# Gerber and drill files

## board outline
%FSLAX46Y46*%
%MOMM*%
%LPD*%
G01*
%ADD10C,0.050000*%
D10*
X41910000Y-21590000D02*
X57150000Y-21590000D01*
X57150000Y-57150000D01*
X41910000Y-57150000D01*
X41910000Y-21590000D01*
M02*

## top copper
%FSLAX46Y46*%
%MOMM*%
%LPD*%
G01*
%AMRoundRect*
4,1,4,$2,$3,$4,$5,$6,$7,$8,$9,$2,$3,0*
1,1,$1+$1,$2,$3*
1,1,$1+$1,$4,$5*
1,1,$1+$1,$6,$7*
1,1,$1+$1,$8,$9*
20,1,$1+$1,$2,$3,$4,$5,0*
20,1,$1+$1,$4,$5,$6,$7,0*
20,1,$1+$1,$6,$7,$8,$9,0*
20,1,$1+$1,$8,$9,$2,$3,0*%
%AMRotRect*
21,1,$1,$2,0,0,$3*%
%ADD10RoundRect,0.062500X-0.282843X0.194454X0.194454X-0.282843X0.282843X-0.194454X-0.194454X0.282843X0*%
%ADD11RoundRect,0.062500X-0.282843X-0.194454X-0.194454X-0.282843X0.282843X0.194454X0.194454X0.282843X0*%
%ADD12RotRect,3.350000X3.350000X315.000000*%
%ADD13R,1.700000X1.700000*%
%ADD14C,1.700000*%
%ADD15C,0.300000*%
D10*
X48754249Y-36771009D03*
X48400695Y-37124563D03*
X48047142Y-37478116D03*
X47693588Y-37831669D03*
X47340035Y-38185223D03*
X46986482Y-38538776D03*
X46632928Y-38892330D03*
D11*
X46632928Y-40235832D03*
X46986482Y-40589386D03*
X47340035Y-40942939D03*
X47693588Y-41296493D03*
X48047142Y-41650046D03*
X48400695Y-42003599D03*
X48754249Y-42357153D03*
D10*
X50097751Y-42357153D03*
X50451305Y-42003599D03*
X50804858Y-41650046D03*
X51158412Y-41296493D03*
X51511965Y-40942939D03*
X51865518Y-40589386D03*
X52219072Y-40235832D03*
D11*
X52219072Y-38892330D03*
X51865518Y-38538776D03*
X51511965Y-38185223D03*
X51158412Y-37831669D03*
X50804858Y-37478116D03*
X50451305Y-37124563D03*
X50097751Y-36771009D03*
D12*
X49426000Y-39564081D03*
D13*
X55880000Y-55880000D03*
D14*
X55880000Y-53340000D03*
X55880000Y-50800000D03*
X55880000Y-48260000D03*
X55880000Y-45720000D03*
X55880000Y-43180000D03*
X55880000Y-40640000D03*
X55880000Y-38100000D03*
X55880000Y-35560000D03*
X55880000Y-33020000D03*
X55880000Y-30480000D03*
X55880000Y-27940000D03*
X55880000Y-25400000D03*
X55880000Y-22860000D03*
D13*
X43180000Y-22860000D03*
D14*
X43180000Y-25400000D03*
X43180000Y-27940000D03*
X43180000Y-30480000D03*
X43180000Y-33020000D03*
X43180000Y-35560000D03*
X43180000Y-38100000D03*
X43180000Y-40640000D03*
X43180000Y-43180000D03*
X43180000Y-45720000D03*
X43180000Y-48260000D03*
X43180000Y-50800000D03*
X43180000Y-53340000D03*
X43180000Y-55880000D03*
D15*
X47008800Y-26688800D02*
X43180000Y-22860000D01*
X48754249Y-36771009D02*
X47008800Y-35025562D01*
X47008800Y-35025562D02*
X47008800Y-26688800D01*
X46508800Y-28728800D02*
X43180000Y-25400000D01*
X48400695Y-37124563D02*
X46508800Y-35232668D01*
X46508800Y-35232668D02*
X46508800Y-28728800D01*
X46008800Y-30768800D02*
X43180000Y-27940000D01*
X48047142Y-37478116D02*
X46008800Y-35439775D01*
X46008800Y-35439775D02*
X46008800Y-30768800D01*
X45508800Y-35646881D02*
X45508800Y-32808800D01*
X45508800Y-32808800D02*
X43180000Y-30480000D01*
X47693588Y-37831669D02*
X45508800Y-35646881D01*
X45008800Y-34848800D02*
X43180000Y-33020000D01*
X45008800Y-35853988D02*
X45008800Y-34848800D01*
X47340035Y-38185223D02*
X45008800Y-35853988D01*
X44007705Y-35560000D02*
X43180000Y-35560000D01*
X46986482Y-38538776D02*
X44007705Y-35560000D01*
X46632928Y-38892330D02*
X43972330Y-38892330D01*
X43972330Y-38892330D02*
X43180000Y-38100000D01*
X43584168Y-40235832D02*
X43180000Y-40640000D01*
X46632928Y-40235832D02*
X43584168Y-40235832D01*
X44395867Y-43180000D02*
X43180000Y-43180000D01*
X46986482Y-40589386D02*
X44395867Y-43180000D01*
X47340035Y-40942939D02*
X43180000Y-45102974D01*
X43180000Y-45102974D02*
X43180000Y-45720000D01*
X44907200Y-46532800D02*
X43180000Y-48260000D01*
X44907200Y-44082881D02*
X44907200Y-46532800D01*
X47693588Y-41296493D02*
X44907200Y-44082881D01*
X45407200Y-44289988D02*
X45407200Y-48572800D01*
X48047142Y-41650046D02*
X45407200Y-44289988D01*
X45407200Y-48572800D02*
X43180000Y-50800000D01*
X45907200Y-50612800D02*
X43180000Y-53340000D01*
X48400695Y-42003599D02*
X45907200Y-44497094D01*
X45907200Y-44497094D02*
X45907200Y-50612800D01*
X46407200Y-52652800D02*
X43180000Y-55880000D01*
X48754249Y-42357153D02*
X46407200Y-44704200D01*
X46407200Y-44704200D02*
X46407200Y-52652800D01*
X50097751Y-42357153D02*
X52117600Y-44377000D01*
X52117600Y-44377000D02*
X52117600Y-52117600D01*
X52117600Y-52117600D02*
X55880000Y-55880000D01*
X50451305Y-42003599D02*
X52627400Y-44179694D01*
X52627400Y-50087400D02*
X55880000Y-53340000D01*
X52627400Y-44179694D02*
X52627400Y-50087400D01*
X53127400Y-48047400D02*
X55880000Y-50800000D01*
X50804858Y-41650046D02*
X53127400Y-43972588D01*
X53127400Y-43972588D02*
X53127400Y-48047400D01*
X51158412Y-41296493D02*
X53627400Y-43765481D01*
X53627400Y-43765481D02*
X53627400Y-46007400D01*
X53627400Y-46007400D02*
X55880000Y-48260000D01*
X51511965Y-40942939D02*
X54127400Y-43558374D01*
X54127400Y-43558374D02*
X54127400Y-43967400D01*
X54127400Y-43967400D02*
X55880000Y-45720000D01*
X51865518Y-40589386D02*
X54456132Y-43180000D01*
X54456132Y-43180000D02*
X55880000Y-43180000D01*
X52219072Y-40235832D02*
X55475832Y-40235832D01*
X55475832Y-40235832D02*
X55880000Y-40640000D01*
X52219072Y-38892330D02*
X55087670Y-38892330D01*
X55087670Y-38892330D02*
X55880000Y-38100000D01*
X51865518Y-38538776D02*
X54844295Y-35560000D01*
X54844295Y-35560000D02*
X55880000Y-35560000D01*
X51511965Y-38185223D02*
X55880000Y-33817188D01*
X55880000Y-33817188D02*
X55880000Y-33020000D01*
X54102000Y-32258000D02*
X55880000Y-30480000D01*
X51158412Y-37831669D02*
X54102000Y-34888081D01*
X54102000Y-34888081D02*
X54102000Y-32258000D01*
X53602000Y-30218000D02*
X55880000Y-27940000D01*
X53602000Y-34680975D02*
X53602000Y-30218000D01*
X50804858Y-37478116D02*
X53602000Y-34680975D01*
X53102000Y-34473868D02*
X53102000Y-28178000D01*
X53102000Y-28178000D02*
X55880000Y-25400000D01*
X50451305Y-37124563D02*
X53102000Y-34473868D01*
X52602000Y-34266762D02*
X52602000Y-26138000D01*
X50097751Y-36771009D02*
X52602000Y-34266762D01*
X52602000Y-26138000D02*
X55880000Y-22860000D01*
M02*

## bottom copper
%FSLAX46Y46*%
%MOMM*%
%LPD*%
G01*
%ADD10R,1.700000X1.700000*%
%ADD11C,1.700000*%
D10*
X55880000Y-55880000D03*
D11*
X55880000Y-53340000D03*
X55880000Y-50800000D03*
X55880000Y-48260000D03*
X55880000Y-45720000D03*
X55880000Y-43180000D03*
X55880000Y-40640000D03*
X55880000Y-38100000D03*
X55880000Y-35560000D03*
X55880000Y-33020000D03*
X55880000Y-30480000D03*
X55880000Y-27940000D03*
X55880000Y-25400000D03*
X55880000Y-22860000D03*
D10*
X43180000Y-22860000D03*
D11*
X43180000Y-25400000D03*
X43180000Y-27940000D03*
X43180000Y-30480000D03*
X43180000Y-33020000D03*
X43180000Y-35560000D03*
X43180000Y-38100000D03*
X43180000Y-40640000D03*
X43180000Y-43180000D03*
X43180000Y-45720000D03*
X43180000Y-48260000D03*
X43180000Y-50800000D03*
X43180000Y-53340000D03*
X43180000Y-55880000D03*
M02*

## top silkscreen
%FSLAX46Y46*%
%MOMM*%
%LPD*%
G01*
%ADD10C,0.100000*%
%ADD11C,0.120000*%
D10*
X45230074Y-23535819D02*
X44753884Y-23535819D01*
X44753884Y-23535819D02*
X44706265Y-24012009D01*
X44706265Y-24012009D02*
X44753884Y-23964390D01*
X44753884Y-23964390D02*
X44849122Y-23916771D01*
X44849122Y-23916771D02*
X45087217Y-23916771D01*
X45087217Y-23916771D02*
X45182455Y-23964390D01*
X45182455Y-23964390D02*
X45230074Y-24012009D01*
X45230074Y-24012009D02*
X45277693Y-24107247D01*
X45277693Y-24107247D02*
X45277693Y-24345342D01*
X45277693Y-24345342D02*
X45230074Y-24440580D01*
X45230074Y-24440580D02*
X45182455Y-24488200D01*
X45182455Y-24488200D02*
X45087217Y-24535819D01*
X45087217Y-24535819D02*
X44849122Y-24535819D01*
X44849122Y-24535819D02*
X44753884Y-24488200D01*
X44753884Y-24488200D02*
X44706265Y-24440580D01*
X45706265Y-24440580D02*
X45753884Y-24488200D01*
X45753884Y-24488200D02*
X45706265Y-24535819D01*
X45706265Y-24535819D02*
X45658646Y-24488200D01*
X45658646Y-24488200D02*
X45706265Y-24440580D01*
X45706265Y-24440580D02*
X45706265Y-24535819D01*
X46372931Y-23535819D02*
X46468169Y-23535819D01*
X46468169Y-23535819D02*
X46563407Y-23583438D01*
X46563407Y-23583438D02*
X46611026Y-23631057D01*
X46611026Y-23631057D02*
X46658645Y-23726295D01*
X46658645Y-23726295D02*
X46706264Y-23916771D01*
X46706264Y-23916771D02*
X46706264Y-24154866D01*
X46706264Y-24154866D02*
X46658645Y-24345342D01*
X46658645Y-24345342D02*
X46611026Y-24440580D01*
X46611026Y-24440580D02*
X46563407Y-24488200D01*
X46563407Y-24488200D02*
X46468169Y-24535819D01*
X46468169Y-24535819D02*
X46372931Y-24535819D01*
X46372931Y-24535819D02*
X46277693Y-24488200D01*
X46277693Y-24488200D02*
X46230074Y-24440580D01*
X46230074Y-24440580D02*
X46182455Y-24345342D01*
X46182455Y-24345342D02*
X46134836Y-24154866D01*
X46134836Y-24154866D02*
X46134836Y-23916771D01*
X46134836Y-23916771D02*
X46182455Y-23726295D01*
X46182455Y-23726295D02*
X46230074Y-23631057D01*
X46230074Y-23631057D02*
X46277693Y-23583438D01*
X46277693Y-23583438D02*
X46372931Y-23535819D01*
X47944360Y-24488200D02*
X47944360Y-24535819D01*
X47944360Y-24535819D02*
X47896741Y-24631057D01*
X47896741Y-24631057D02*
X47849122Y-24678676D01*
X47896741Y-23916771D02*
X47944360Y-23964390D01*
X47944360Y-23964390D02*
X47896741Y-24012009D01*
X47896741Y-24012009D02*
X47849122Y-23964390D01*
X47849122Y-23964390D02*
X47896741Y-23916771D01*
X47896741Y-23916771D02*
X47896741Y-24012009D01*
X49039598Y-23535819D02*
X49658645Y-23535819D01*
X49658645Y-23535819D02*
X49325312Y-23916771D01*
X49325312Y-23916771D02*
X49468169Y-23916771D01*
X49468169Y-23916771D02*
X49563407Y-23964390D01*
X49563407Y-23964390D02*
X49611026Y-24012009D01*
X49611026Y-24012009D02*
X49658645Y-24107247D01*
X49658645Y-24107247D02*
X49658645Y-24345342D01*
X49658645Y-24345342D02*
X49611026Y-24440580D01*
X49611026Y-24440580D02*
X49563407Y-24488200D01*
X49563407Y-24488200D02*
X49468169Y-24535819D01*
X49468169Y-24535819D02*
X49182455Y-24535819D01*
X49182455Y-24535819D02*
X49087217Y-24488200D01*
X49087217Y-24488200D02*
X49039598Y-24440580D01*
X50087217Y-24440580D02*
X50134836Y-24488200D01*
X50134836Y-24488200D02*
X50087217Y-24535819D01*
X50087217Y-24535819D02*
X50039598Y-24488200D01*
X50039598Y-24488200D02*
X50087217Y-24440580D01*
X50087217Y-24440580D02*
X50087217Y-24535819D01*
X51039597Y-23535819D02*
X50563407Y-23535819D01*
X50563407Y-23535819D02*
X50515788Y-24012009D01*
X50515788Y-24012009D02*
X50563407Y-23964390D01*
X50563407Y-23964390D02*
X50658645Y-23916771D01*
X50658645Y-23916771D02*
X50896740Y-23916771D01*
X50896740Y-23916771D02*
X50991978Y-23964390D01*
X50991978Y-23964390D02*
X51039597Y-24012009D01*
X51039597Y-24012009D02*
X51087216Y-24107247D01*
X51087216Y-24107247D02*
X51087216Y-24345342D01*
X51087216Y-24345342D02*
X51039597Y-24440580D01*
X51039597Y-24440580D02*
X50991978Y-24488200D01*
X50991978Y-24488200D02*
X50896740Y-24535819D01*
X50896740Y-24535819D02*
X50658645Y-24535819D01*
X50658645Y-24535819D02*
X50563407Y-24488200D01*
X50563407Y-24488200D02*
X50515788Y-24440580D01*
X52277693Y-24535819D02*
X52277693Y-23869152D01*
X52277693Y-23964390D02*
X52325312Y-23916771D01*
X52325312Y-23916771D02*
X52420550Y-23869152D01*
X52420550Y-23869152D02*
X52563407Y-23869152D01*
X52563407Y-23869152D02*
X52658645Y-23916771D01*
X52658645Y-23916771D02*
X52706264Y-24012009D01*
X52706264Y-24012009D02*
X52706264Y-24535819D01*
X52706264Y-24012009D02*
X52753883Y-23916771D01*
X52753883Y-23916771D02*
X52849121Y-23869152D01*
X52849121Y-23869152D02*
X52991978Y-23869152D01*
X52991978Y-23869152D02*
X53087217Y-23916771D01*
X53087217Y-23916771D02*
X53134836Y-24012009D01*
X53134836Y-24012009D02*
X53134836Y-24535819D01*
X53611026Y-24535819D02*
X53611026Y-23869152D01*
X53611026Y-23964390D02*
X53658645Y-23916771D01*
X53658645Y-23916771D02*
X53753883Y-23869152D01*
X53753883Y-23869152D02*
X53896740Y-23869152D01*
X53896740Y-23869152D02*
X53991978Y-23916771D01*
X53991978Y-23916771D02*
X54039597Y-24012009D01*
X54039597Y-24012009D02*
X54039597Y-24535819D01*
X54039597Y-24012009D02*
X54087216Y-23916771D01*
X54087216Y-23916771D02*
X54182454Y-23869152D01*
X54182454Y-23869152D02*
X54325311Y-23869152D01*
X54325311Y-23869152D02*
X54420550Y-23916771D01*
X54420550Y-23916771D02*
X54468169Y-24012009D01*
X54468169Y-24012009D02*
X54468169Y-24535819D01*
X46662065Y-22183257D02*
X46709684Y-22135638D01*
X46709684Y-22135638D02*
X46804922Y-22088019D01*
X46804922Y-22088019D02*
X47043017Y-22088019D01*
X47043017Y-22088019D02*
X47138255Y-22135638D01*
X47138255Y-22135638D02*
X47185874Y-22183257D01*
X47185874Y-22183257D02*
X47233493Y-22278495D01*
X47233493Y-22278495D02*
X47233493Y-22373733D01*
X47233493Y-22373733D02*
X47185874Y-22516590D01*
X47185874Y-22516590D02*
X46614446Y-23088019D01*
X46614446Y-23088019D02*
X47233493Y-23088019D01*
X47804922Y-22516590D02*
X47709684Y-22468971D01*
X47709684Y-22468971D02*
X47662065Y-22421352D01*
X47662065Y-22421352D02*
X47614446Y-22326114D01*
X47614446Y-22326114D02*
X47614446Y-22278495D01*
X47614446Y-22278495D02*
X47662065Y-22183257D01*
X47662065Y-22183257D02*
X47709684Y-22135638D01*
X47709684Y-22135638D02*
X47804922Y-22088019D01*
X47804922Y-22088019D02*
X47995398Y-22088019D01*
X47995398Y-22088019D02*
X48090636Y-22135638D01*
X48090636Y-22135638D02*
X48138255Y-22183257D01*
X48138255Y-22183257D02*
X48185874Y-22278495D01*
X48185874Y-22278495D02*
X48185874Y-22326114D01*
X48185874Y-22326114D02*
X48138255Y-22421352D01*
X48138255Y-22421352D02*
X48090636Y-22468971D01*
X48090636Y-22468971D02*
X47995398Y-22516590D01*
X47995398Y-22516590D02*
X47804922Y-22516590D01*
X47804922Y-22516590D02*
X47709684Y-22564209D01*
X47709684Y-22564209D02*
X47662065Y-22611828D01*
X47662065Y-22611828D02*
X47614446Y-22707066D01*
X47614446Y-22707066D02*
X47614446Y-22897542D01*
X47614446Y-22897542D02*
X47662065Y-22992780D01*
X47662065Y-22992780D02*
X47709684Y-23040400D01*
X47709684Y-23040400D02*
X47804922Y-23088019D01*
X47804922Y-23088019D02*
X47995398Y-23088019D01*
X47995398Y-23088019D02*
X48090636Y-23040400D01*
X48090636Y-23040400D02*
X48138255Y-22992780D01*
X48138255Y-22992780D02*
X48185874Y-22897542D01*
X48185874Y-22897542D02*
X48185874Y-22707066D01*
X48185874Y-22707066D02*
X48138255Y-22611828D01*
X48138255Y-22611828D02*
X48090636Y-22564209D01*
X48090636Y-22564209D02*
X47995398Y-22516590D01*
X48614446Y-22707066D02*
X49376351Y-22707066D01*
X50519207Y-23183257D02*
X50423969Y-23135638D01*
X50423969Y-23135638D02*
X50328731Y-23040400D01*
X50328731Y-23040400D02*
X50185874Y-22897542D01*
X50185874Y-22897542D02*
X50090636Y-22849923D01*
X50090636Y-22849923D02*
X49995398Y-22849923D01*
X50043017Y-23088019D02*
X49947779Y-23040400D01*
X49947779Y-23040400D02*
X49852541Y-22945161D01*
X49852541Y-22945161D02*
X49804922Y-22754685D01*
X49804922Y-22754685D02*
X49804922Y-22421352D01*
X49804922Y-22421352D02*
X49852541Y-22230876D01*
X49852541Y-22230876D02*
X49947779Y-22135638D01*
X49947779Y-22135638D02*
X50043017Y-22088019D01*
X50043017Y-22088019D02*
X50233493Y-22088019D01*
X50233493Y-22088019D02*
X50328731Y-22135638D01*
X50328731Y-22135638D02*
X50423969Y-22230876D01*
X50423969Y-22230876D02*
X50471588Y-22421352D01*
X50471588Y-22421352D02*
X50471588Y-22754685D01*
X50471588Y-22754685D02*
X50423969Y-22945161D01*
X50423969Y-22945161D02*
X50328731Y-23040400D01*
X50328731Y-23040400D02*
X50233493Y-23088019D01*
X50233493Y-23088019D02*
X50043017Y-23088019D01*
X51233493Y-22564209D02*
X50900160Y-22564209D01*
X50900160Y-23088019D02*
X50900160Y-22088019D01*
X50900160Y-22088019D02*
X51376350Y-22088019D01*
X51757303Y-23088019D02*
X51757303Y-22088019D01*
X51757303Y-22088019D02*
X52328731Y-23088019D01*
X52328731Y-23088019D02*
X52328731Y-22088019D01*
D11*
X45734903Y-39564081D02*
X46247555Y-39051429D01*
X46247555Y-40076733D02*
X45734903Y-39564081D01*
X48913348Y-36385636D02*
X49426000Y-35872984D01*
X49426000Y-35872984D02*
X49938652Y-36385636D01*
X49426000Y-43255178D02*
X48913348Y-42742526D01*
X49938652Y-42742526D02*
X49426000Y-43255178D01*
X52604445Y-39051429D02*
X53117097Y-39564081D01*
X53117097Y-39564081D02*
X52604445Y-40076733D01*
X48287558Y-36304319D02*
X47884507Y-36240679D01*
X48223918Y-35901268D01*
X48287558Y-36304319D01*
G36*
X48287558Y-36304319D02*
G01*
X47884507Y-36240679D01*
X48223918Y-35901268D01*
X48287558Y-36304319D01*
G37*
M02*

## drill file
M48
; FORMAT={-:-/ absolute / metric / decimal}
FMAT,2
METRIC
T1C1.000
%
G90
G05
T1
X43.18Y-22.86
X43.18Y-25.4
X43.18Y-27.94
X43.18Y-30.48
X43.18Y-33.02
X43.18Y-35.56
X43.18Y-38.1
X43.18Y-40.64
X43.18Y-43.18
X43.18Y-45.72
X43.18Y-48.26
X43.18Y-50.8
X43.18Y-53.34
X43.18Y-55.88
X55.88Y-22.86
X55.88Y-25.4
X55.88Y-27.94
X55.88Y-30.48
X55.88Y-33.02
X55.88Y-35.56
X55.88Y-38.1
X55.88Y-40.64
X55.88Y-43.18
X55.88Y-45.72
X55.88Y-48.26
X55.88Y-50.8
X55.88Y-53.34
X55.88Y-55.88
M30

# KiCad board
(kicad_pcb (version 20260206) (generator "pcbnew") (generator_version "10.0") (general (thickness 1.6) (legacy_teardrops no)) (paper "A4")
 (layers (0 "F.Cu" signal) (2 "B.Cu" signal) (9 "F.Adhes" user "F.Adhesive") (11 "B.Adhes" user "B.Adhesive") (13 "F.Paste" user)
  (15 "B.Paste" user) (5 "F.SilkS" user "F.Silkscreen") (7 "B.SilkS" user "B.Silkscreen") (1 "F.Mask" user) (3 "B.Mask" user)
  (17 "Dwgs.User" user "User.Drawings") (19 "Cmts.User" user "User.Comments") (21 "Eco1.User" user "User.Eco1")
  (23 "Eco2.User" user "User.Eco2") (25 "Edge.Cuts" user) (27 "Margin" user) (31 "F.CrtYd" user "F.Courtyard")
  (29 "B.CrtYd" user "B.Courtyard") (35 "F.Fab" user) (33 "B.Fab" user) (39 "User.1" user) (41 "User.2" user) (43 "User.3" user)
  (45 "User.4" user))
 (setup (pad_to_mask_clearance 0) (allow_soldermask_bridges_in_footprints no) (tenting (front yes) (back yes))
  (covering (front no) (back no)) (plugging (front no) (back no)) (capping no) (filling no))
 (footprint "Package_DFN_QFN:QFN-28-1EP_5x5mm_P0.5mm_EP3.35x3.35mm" (layer "F.Cu") (at 49.426 39.564081 -45)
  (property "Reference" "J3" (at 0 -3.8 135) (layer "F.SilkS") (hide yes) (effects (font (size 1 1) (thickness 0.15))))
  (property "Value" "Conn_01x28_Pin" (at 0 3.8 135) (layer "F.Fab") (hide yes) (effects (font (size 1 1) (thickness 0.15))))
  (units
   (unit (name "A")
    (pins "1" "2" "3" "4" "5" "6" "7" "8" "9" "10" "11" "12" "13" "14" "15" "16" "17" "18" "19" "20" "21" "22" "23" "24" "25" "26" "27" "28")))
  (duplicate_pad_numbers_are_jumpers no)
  (fp_line (start -2.61 2.61) (end -2.61 1.885) (stroke (width 0.12) (type solid)) (layer "F.SilkS"))
  (fp_line (start -1.885 2.61) (end -2.61 2.61) (stroke (width 0.12) (type solid)) (layer "F.SilkS"))
  (fp_line (start -2.61 -1.885) (end -2.61 -2.61) (stroke (width 0.12) (type solid)) (layer "F.SilkS"))
  (fp_line (start -2.61 -2.61) (end -1.885 -2.61) (stroke (width 0.12) (type solid)) (layer "F.SilkS"))
  (fp_line (start 2.61 2.61) (end 1.885 2.61) (stroke (width 0.12) (type solid)) (layer "F.SilkS"))
  (fp_line (start 2.61 1.885) (end 2.61 2.61) (stroke (width 0.12) (type solid)) (layer "F.SilkS"))
  (fp_line (start 1.885 -2.61) (end 2.61 -2.61) (stroke (width 0.12) (type solid)) (layer "F.SilkS"))
  (fp_line (start 2.61 -2.61) (end 2.61 -1.885) (stroke (width 0.12) (type solid)) (layer "F.SilkS"))
  (fp_poly (pts (xy -3.11 -1.5) (xy -3.44 -1.26) (xy -3.44 -1.74)) (stroke (width 0.12) (type solid)) (fill yes) (layer "F.SilkS"))
  (pad "" smd roundrect (at -1.120001 0 315) (size 0.9 0.9) (layers "F.Paste") (roundrect_rratio 0.25))
  (pad "" smd roundrect (at -1.12 -1.12 315) (size 0.9 0.9) (layers "F.Paste") (roundrect_rratio 0.25))
  (pad "" smd roundrect (at -1.12 1.12 315) (size 0.9 0.9) (layers "F.Paste") (roundrect_rratio 0.25))
  (pad "" smd roundrect (at 0 -1.120001 315) (size 0.9 0.9) (layers "F.Paste") (roundrect_rratio 0.25))
  (pad "" smd roundrect (at 0 0 315) (size 0.9 0.9) (layers "F.Paste") (roundrect_rratio 0.25))
  (pad "" smd roundrect (at 0 1.120001 315) (size 0.9 0.9) (layers "F.Paste") (roundrect_rratio 0.25))
  (pad "" smd roundrect (at 1.12 -1.12 315) (size 0.9 0.9) (layers "F.Paste") (roundrect_rratio 0.25))
  (pad "" smd roundrect (at 1.12 1.12 315) (size 0.9 0.9) (layers "F.Paste") (roundrect_rratio 0.25))
  (pad "" smd roundrect (at 1.120001 0 315) (size 0.9 0.9) (layers "F.Paste") (roundrect_rratio 0.25))
  (pad "1" smd roundrect (at -2.45 -1.5 315) (size 0.8 0.25) (layers "F.Cu" "F.Mask" "F.Paste") (roundrect_rratio 0.25)
   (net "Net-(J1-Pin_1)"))
  (pad "2" smd roundrect (at -2.45 -1 315) (size 0.8 0.25) (layers "F.Cu" "F.Mask" "F.Paste") (roundrect_rratio 0.25) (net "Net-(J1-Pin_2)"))
  (pad "3" smd roundrect (at -2.45 -0.5 315) (size 0.8 0.25) (layers "F.Cu" "F.Mask" "F.Paste") (roundrect_rratio 0.25)
   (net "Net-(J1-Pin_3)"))
  (pad "4" smd roundrect (at -2.450001 0 315) (size 0.8 0.25) (layers "F.Cu" "F.Mask" "F.Paste") (roundrect_rratio 0.25)
   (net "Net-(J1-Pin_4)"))
  (pad "5" smd roundrect (at -2.45 0.5 315) (size 0.8 0.25) (layers "F.Cu" "F.Mask" "F.Paste") (roundrect_rratio 0.25)
   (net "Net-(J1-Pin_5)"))
  (pad "6" smd roundrect (at -2.45 1 315) (size 0.8 0.25) (layers "F.Cu" "F.Mask" "F.Paste") (roundrect_rratio 0.25) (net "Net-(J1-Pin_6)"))
  (pad "7" smd roundrect (at -2.45 1.5 315) (size 0.8 0.25) (layers "F.Cu" "F.Mask" "F.Paste") (roundrect_rratio 0.25)
   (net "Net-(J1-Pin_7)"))
  (pad "8" smd roundrect (at -1.5 2.45 315) (size 0.25 0.8) (layers "F.Cu" "F.Mask" "F.Paste") (roundrect_rratio 0.25)
   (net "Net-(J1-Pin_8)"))
  (pad "9" smd roundrect (at -1 2.45 315) (size 0.25 0.8) (layers "F.Cu" "F.Mask" "F.Paste") (roundrect_rratio 0.25) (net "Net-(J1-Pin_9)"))
  (pad "10" smd roundrect (at -0.5 2.45 315) (size 0.25 0.8) (layers "F.Cu" "F.Mask" "F.Paste") (roundrect_rratio 0.25)
   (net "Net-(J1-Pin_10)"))
  (pad "11" smd roundrect (at 0 2.450001 315) (size 0.25 0.8) (layers "F.Cu" "F.Mask" "F.Paste") (roundrect_rratio 0.25)
   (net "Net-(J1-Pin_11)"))
  (pad "12" smd roundrect (at 0.5 2.45 315) (size 0.25 0.8) (layers "F.Cu" "F.Mask" "F.Paste") (roundrect_rratio 0.25)
   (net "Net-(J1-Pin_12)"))
  (pad "13" smd roundrect (at 1 2.45 315) (size 0.25 0.8) (layers "F.Cu" "F.Mask" "F.Paste") (roundrect_rratio 0.25) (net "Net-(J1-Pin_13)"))
  (pad "14" smd roundrect (at 1.5 2.45 315) (size 0.25 0.8) (layers "F.Cu" "F.Mask" "F.Paste") (roundrect_rratio 0.25)
   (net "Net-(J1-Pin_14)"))
  (pad "15" smd roundrect (at 2.45 1.5 315) (size 0.8 0.25) (layers "F.Cu" "F.Mask" "F.Paste") (roundrect_rratio 0.25)
   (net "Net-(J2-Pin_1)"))
  (pad "16" smd roundrect (at 2.45 1 315) (size 0.8 0.25) (layers "F.Cu" "F.Mask" "F.Paste") (roundrect_rratio 0.25) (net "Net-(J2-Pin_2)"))
  (pad "17" smd roundrect (at 2.45 0.5 315) (size 0.8 0.25) (layers "F.Cu" "F.Mask" "F.Paste") (roundrect_rratio 0.25)
   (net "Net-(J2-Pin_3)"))
  (pad "18" smd roundrect (at 2.450001 0 315) (size 0.8 0.25) (layers "F.Cu" "F.Mask" "F.Paste") (roundrect_rratio 0.25)
   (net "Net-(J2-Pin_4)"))
  (pad "19" smd roundrect (at 2.45 -0.5 315) (size 0.8 0.25) (layers "F.Cu" "F.Mask" "F.Paste") (roundrect_rratio 0.25)
   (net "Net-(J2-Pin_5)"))
  (pad "20" smd roundrect (at 2.45 -1 315) (size 0.8 0.25) (layers "F.Cu" "F.Mask" "F.Paste") (roundrect_rratio 0.25) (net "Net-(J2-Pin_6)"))
  (pad "21" smd roundrect (at 2.45 -1.5 315) (size 0.8 0.25) (layers "F.Cu" "F.Mask" "F.Paste") (roundrect_rratio 0.25)
   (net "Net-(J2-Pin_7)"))
  (pad "22" smd roundrect (at 1.5 -2.45 315) (size 0.25 0.8) (layers "F.Cu" "F.Mask" "F.Paste") (roundrect_rratio 0.25)
   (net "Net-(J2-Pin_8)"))
  (pad "23" smd roundrect (at 1 -2.45 315) (size 0.25 0.8) (layers "F.Cu" "F.Mask" "F.Paste") (roundrect_rratio 0.25) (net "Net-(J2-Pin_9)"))
  (pad "24" smd roundrect (at 0.5 -2.45 315) (size 0.25 0.8) (layers "F.Cu" "F.Mask" "F.Paste") (roundrect_rratio 0.25)
   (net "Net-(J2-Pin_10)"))
  (pad "25" smd roundrect (at 0 -2.450001 315) (size 0.25 0.8) (layers "F.Cu" "F.Mask" "F.Paste") (roundrect_rratio 0.25)
   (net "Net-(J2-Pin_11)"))
  (pad "26" smd roundrect (at -0.5 -2.45 315) (size 0.25 0.8) (layers "F.Cu" "F.Mask" "F.Paste") (roundrect_rratio 0.25)
   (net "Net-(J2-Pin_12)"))
  (pad "27" smd roundrect (at -1 -2.45 315) (size 0.25 0.8) (layers "F.Cu" "F.Mask" "F.Paste") (roundrect_rratio 0.25)
   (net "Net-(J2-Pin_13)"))
  (pad "28" smd roundrect (at -1.5 -2.45 315) (size 0.25 0.8) (layers "F.Cu" "F.Mask" "F.Paste") (roundrect_rratio 0.25)
   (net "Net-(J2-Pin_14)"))
  (pad "29" smd rect (at 0 0 315) (size 3.35 3.35) (layers "F.Cu" "F.Mask") (zone_connect 2)))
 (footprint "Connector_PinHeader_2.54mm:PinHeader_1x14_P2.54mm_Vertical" (layer "B.Cu") (at 55.88 55.88)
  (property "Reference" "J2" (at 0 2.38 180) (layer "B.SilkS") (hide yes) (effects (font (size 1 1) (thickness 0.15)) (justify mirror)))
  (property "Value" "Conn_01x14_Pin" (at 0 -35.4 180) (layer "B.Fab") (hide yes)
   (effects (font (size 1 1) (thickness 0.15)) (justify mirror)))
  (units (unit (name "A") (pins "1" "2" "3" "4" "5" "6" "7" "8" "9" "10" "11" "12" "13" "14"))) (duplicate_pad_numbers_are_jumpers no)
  (pad "1" thru_hole rect (at 0 0) (size 1.7 1.7) (drill 1) (layers "*.Cu" "*.Mask") (remove_unused_layers no) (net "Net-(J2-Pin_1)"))
  (pad "2" thru_hole circle (at 0 -2.54) (size 1.7 1.7) (drill 1) (layers "*.Cu" "*.Mask") (remove_unused_layers no) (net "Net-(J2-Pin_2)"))
  (pad "3" thru_hole circle (at 0 -5.08) (size 1.7 1.7) (drill 1) (layers "*.Cu" "*.Mask") (remove_unused_layers no) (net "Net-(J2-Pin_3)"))
  (pad "4" thru_hole circle (at 0 -7.62) (size 1.7 1.7) (drill 1) (layers "*.Cu" "*.Mask") (remove_unused_layers no) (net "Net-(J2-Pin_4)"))
  (pad "5" thru_hole circle (at 0 -10.16) (size 1.7 1.7) (drill 1) (layers "*.Cu" "*.Mask") (remove_unused_layers no) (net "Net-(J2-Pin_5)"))
  (pad "6" thru_hole circle (at 0 -12.7) (size 1.7 1.7) (drill 1) (layers "*.Cu" "*.Mask") (remove_unused_layers no) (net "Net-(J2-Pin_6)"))
  (pad "7" thru_hole circle (at 0 -15.24) (size 1.7 1.7) (drill 1) (layers "*.Cu" "*.Mask") (remove_unused_layers no) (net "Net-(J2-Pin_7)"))
  (pad "8" thru_hole circle (at 0 -17.78) (size 1.7 1.7) (drill 1) (layers "*.Cu" "*.Mask") (remove_unused_layers no) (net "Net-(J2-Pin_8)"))
  (pad "9" thru_hole circle (at 0 -20.32) (size 1.7 1.7) (drill 1) (layers "*.Cu" "*.Mask") (remove_unused_layers no) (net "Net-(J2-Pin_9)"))
  (pad "10" thru_hole circle (at 0 -22.86) (size 1.7 1.7) (drill 1) (layers "*.Cu" "*.Mask") (remove_unused_layers no)
   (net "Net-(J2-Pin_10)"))
  (pad "11" thru_hole circle (at 0 -25.4) (size 1.7 1.7) (drill 1) (layers "*.Cu" "*.Mask") (remove_unused_layers no)
   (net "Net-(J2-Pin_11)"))
  (pad "12" thru_hole circle (at 0 -27.94) (size 1.7 1.7) (drill 1) (layers "*.Cu" "*.Mask") (remove_unused_layers no)
   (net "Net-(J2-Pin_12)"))
  (pad "13" thru_hole circle (at 0 -30.48) (size 1.7 1.7) (drill 1) (layers "*.Cu" "*.Mask") (remove_unused_layers no)
   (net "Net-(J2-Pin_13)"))
  (pad "14" thru_hole circle (at 0 -33.02) (size 1.7 1.7) (drill 1) (layers "*.Cu" "*.Mask") (remove_unused_layers no)
   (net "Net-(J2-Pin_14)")))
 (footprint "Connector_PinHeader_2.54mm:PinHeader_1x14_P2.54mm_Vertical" (layer "B.Cu") (at 43.18 22.86 180)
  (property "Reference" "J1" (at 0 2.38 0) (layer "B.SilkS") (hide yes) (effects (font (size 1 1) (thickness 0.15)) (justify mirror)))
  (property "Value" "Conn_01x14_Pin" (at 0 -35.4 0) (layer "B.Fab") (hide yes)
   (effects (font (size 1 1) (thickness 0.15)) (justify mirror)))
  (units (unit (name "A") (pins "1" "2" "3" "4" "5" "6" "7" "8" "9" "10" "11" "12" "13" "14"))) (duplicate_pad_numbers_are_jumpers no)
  (pad "1" thru_hole rect (at 0 0 180) (size 1.7 1.7) (drill 1) (layers "*.Cu" "*.Mask") (remove_unused_layers no) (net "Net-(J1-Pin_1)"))
  (pad "2" thru_hole circle (at 0 -2.54 180) (size 1.7 1.7) (drill 1) (layers "*.Cu" "*.Mask") (remove_unused_layers no)
   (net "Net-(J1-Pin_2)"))
  (pad "3" thru_hole circle (at 0 -5.08 180) (size 1.7 1.7) (drill 1) (layers "*.Cu" "*.Mask") (remove_unused_layers no)
   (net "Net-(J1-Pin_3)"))
  (pad "4" thru_hole circle (at 0 -7.62 180) (size 1.7 1.7) (drill 1) (layers "*.Cu" "*.Mask") (remove_unused_layers no)
   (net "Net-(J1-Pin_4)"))
  (pad "5" thru_hole circle (at 0 -10.16 180) (size 1.7 1.7) (drill 1) (layers "*.Cu" "*.Mask") (remove_unused_layers no)
   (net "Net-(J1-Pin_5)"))
  (pad "6" thru_hole circle (at 0 -12.7 180) (size 1.7 1.7) (drill 1) (layers "*.Cu" "*.Mask") (remove_unused_layers no)
   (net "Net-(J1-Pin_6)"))
  (pad "7" thru_hole circle (at 0 -15.24 180) (size 1.7 1.7) (drill 1) (layers "*.Cu" "*.Mask") (remove_unused_layers no)
   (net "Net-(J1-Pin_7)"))
  (pad "8" thru_hole circle (at 0 -17.78 180) (size 1.7 1.7) (drill 1) (layers "*.Cu" "*.Mask") (remove_unused_layers no)
   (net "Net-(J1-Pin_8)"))
  (pad "9" thru_hole circle (at 0 -20.32 180) (size 1.7 1.7) (drill 1) (layers "*.Cu" "*.Mask") (remove_unused_layers no)
   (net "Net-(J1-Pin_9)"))
  (pad "10" thru_hole circle (at 0 -22.86 180) (size 1.7 1.7) (drill 1) (layers "*.Cu" "*.Mask") (remove_unused_layers no)
   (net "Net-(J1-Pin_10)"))
  (pad "11" thru_hole circle (at 0 -25.4 180) (size 1.7 1.7) (drill 1) (layers "*.Cu" "*.Mask") (remove_unused_layers no)
   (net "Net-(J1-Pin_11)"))
  (pad "12" thru_hole circle (at 0 -27.94 180) (size 1.7 1.7) (drill 1) (layers "*.Cu" "*.Mask") (remove_unused_layers no)
   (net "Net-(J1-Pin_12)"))
  (pad "13" thru_hole circle (at 0 -30.48 180) (size 1.7 1.7) (drill 1) (layers "*.Cu" "*.Mask") (remove_unused_layers no)
   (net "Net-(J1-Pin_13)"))
  (pad "14" thru_hole circle (at 0 -33.02 180) (size 1.7 1.7) (drill 1) (layers "*.Cu" "*.Mask") (remove_unused_layers no)
   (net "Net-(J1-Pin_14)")))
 (gr_rect (start 41.91 21.59) (end 57.15 57.15) (stroke (width 0.05) (type default)) (fill no) (layer "Edge.Cuts"))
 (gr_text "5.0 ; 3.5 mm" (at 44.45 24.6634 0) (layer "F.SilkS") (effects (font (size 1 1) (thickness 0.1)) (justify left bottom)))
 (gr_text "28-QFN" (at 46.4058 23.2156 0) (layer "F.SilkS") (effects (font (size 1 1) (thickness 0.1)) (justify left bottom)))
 (segment (start 47.0088 26.6888) (end 43.18 22.86) (width 0.3) (layer "F.Cu") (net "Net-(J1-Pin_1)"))
 (segment (start 48.754249 36.771009) (end 47.0088 35.025562) (width 0.3) (layer "F.Cu") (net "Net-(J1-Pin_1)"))
 (segment (start 47.0088 35.025562) (end 47.0088 26.6888) (width 0.3) (layer "F.Cu") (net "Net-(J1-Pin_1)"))
 (segment (start 46.5088 28.7288) (end 43.18 25.4) (width 0.3) (layer "F.Cu") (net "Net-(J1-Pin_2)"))
 (segment (start 48.400695 37.124563) (end 46.5088 35.232668) (width 0.3) (layer "F.Cu") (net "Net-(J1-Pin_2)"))
 (segment (start 46.5088 35.232668) (end 46.5088 28.7288) (width 0.3) (layer "F.Cu") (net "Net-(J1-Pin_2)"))
 (segment (start 46.0088 30.7688) (end 43.18 27.94) (width 0.3) (layer "F.Cu") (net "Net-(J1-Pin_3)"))
 (segment (start 48.047142 37.478116) (end 46.0088 35.439775) (width 0.3) (layer "F.Cu") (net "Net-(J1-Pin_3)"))
 (segment (start 46.0088 35.439775) (end 46.0088 30.7688) (width 0.3) (layer "F.Cu") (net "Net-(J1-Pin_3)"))
 (segment (start 45.5088 35.646881) (end 45.5088 32.8088) (width 0.3) (layer "F.Cu") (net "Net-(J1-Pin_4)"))
 (segment (start 45.5088 32.8088) (end 43.18 30.48) (width 0.3) (layer "F.Cu") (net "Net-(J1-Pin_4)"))
 (segment (start 47.693588 37.831669) (end 45.5088 35.646881) (width 0.3) (layer "F.Cu") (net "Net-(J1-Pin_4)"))
 (segment (start 45.0088 34.8488) (end 43.18 33.02) (width 0.3) (layer "F.Cu") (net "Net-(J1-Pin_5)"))
 (segment (start 45.0088 35.853988) (end 45.0088 34.8488) (width 0.3) (layer "F.Cu") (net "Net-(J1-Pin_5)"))
 (segment (start 47.340035 38.185223) (end 45.0088 35.853988) (width 0.3) (layer "F.Cu") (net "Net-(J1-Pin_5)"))
 (segment (start 44.007705 35.56) (end 43.18 35.56) (width 0.3) (layer "F.Cu") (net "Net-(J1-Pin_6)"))
 (segment (start 46.986482 38.538776) (end 44.007705 35.56) (width 0.3) (layer "F.Cu") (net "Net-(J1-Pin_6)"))
 (segment (start 46.632928 38.89233) (end 43.97233 38.89233) (width 0.3) (layer "F.Cu") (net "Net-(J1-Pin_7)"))
 (segment (start 43.97233 38.89233) (end 43.18 38.1) (width 0.3) (layer "F.Cu") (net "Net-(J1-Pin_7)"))
 (segment (start 43.584168 40.235832) (end 43.18 40.64) (width 0.3) (layer "F.Cu") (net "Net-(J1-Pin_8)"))
 (segment (start 46.632928 40.235832) (end 43.584168 40.235832) (width 0.3) (layer "F.Cu") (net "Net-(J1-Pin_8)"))
 (segment (start 44.395867 43.18) (end 43.18 43.18) (width 0.3) (layer "F.Cu") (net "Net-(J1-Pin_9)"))
 (segment (start 46.986482 40.589386) (end 44.395867 43.18) (width 0.3) (layer "F.Cu") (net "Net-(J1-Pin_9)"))
 (segment (start 47.340035 40.942939) (end 43.18 45.102974) (width 0.3) (layer "F.Cu") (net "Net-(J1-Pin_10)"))
 (segment (start 43.18 45.102974) (end 43.18 45.72) (width 0.3) (layer "F.Cu") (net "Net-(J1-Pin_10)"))
 (segment (start 44.9072 46.5328) (end 43.18 48.26) (width 0.3) (layer "F.Cu") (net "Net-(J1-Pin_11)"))
 (segment (start 44.9072 44.082881) (end 44.9072 46.5328) (width 0.3) (layer "F.Cu") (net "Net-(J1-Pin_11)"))
 (segment (start 47.693588 41.296493) (end 44.9072 44.082881) (width 0.3) (layer "F.Cu") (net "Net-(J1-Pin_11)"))
 (segment (start 45.4072 44.289988) (end 45.4072 48.5728) (width 0.3) (layer "F.Cu") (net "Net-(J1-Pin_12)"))
 (segment (start 48.047142 41.650046) (end 45.4072 44.289988) (width 0.3) (layer "F.Cu") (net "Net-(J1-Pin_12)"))
 (segment (start 45.4072 48.5728) (end 43.18 50.8) (width 0.3) (layer "F.Cu") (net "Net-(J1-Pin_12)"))
 (segment (start 45.9072 50.6128) (end 43.18 53.34) (width 0.3) (layer "F.Cu") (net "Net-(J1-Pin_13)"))
 (segment (start 48.400695 42.003599) (end 45.9072 44.497094) (width 0.3) (layer "F.Cu") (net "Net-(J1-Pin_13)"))
 (segment (start 45.9072 44.497094) (end 45.9072 50.6128) (width 0.3) (layer "F.Cu") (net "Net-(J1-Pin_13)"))
 (segment (start 46.4072 52.6528) (end 43.18 55.88) (width 0.3) (layer "F.Cu") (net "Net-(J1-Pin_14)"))
 (segment (start 48.754249 42.357153) (end 46.4072 44.7042) (width 0.3) (layer "F.Cu") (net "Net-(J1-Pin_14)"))
 (segment (start 46.4072 44.7042) (end 46.4072 52.6528) (width 0.3) (layer "F.Cu") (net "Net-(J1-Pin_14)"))
 (segment (start 50.097751 42.357153) (end 52.1176 44.377) (width 0.3) (layer "F.Cu") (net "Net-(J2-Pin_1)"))
 (segment (start 52.1176 44.377) (end 52.1176 52.1176) (width 0.3) (layer "F.Cu") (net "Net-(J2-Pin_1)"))
 (segment (start 52.1176 52.1176) (end 55.88 55.88) (width 0.3) (layer "F.Cu") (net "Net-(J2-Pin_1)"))
 (segment (start 50.451305 42.003599) (end 52.6274 44.179694) (width 0.3) (layer "F.Cu") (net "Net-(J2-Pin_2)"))
 (segment (start 52.6274 50.0874) (end 55.88 53.34) (width 0.3) (layer "F.Cu") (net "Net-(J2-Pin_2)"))
 (segment (start 52.6274 44.179694) (end 52.6274 50.0874) (width 0.3) (layer "F.Cu") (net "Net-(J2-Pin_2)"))
 (segment (start 53.1274 48.0474) (end 55.88 50.8) (width 0.3) (layer "F.Cu") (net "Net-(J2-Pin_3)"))
 (segment (start 50.804858 41.650046) (end 53.1274 43.972588) (width 0.3) (layer "F.Cu") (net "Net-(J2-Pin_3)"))
 (segment (start 53.1274 43.972588) (end 53.1274 48.0474) (width 0.3) (layer "F.Cu") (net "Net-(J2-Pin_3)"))
 (segment (start 51.158412 41.296493) (end 53.6274 43.765481) (width 0.3) (layer "F.Cu") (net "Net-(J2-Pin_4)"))
 (segment (start 53.6274 43.765481) (end 53.6274 46.0074) (width 0.3) (layer "F.Cu") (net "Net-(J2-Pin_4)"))
 (segment (start 53.6274 46.0074) (end 55.88 48.26) (width 0.3) (layer "F.Cu") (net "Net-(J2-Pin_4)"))
 (segment (start 51.511965 40.942939) (end 54.1274 43.558374) (width 0.3) (layer "F.Cu") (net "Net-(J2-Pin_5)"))
 (segment (start 54.1274 43.558374) (end 54.1274 43.9674) (width 0.3) (layer "F.Cu") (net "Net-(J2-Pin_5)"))
 (segment (start 54.1274 43.9674) (end 55.88 45.72) (width 0.3) (layer "F.Cu") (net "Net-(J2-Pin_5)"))
 (segment (start 51.865518 40.589386) (end 54.456132 43.18) (width 0.3) (layer "F.Cu") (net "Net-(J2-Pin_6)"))
 (segment (start 54.456132 43.18) (end 55.88 43.18) (width 0.3) (layer "F.Cu") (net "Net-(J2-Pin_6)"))
 (segment (start 52.219072 40.235832) (end 55.475832 40.235832) (width 0.3) (layer "F.Cu") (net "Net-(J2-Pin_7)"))
 (segment (start 55.475832 40.235832) (end 55.88 40.64) (width 0.3) (layer "F.Cu") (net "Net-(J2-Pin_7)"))
 (segment (start 52.219072 38.89233) (end 55.08767 38.89233) (width 0.3) (layer "F.Cu") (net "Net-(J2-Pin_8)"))
 (segment (start 55.08767 38.89233) (end 55.88 38.1) (width 0.3) (layer "F.Cu") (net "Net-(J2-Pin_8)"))
 (segment (start 51.865518 38.538776) (end 54.844295 35.56) (width 0.3) (layer "F.Cu") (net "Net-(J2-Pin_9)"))
 (segment (start 54.844295 35.56) (end 55.88 35.56) (width 0.3) (layer "F.Cu") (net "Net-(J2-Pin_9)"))
 (segment (start 51.511965 38.185223) (end 55.88 33.817188) (width 0.3) (layer "F.Cu") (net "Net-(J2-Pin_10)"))
 (segment (start 55.88 33.817188) (end 55.88 33.02) (width 0.3) (layer "F.Cu") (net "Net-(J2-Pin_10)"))
 (segment (start 54.102 32.258) (end 55.88 30.48) (width 0.3) (layer "F.Cu") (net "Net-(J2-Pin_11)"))
 (segment (start 51.158412 37.831669) (end 54.102 34.888081) (width 0.3) (layer "F.Cu") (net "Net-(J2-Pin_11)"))
 (segment (start 54.102 34.888081) (end 54.102 32.258) (width 0.3) (layer "F.Cu") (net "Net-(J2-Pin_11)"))
 (segment (start 53.602 30.218) (end 55.88 27.94) (width 0.3) (layer "F.Cu") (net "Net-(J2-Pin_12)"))
 (segment (start 53.602 34.680975) (end 53.602 30.218) (width 0.3) (layer "F.Cu") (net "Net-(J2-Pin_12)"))
 (segment (start 50.804858 37.478116) (end 53.602 34.680975) (width 0.3) (layer "F.Cu") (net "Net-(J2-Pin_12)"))
 (segment (start 53.102 34.473868) (end 53.102 28.178) (width 0.3) (layer "F.Cu") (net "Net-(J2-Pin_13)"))
 (segment (start 53.102 28.178) (end 55.88 25.4) (width 0.3) (layer "F.Cu") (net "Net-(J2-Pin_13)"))
 (segment (start 50.451305 37.124563) (end 53.102 34.473868) (width 0.3) (layer "F.Cu") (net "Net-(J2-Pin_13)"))
 (segment (start 52.602 34.266762) (end 52.602 26.138) (width 0.3) (layer "F.Cu") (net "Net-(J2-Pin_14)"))
 (segment (start 50.097751 36.771009) (end 52.602 34.266762) (width 0.3) (layer "F.Cu") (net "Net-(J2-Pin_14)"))
 (segment (start 52.602 26.138) (end 55.88 22.86) (width 0.3) (layer "F.Cu") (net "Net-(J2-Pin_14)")))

